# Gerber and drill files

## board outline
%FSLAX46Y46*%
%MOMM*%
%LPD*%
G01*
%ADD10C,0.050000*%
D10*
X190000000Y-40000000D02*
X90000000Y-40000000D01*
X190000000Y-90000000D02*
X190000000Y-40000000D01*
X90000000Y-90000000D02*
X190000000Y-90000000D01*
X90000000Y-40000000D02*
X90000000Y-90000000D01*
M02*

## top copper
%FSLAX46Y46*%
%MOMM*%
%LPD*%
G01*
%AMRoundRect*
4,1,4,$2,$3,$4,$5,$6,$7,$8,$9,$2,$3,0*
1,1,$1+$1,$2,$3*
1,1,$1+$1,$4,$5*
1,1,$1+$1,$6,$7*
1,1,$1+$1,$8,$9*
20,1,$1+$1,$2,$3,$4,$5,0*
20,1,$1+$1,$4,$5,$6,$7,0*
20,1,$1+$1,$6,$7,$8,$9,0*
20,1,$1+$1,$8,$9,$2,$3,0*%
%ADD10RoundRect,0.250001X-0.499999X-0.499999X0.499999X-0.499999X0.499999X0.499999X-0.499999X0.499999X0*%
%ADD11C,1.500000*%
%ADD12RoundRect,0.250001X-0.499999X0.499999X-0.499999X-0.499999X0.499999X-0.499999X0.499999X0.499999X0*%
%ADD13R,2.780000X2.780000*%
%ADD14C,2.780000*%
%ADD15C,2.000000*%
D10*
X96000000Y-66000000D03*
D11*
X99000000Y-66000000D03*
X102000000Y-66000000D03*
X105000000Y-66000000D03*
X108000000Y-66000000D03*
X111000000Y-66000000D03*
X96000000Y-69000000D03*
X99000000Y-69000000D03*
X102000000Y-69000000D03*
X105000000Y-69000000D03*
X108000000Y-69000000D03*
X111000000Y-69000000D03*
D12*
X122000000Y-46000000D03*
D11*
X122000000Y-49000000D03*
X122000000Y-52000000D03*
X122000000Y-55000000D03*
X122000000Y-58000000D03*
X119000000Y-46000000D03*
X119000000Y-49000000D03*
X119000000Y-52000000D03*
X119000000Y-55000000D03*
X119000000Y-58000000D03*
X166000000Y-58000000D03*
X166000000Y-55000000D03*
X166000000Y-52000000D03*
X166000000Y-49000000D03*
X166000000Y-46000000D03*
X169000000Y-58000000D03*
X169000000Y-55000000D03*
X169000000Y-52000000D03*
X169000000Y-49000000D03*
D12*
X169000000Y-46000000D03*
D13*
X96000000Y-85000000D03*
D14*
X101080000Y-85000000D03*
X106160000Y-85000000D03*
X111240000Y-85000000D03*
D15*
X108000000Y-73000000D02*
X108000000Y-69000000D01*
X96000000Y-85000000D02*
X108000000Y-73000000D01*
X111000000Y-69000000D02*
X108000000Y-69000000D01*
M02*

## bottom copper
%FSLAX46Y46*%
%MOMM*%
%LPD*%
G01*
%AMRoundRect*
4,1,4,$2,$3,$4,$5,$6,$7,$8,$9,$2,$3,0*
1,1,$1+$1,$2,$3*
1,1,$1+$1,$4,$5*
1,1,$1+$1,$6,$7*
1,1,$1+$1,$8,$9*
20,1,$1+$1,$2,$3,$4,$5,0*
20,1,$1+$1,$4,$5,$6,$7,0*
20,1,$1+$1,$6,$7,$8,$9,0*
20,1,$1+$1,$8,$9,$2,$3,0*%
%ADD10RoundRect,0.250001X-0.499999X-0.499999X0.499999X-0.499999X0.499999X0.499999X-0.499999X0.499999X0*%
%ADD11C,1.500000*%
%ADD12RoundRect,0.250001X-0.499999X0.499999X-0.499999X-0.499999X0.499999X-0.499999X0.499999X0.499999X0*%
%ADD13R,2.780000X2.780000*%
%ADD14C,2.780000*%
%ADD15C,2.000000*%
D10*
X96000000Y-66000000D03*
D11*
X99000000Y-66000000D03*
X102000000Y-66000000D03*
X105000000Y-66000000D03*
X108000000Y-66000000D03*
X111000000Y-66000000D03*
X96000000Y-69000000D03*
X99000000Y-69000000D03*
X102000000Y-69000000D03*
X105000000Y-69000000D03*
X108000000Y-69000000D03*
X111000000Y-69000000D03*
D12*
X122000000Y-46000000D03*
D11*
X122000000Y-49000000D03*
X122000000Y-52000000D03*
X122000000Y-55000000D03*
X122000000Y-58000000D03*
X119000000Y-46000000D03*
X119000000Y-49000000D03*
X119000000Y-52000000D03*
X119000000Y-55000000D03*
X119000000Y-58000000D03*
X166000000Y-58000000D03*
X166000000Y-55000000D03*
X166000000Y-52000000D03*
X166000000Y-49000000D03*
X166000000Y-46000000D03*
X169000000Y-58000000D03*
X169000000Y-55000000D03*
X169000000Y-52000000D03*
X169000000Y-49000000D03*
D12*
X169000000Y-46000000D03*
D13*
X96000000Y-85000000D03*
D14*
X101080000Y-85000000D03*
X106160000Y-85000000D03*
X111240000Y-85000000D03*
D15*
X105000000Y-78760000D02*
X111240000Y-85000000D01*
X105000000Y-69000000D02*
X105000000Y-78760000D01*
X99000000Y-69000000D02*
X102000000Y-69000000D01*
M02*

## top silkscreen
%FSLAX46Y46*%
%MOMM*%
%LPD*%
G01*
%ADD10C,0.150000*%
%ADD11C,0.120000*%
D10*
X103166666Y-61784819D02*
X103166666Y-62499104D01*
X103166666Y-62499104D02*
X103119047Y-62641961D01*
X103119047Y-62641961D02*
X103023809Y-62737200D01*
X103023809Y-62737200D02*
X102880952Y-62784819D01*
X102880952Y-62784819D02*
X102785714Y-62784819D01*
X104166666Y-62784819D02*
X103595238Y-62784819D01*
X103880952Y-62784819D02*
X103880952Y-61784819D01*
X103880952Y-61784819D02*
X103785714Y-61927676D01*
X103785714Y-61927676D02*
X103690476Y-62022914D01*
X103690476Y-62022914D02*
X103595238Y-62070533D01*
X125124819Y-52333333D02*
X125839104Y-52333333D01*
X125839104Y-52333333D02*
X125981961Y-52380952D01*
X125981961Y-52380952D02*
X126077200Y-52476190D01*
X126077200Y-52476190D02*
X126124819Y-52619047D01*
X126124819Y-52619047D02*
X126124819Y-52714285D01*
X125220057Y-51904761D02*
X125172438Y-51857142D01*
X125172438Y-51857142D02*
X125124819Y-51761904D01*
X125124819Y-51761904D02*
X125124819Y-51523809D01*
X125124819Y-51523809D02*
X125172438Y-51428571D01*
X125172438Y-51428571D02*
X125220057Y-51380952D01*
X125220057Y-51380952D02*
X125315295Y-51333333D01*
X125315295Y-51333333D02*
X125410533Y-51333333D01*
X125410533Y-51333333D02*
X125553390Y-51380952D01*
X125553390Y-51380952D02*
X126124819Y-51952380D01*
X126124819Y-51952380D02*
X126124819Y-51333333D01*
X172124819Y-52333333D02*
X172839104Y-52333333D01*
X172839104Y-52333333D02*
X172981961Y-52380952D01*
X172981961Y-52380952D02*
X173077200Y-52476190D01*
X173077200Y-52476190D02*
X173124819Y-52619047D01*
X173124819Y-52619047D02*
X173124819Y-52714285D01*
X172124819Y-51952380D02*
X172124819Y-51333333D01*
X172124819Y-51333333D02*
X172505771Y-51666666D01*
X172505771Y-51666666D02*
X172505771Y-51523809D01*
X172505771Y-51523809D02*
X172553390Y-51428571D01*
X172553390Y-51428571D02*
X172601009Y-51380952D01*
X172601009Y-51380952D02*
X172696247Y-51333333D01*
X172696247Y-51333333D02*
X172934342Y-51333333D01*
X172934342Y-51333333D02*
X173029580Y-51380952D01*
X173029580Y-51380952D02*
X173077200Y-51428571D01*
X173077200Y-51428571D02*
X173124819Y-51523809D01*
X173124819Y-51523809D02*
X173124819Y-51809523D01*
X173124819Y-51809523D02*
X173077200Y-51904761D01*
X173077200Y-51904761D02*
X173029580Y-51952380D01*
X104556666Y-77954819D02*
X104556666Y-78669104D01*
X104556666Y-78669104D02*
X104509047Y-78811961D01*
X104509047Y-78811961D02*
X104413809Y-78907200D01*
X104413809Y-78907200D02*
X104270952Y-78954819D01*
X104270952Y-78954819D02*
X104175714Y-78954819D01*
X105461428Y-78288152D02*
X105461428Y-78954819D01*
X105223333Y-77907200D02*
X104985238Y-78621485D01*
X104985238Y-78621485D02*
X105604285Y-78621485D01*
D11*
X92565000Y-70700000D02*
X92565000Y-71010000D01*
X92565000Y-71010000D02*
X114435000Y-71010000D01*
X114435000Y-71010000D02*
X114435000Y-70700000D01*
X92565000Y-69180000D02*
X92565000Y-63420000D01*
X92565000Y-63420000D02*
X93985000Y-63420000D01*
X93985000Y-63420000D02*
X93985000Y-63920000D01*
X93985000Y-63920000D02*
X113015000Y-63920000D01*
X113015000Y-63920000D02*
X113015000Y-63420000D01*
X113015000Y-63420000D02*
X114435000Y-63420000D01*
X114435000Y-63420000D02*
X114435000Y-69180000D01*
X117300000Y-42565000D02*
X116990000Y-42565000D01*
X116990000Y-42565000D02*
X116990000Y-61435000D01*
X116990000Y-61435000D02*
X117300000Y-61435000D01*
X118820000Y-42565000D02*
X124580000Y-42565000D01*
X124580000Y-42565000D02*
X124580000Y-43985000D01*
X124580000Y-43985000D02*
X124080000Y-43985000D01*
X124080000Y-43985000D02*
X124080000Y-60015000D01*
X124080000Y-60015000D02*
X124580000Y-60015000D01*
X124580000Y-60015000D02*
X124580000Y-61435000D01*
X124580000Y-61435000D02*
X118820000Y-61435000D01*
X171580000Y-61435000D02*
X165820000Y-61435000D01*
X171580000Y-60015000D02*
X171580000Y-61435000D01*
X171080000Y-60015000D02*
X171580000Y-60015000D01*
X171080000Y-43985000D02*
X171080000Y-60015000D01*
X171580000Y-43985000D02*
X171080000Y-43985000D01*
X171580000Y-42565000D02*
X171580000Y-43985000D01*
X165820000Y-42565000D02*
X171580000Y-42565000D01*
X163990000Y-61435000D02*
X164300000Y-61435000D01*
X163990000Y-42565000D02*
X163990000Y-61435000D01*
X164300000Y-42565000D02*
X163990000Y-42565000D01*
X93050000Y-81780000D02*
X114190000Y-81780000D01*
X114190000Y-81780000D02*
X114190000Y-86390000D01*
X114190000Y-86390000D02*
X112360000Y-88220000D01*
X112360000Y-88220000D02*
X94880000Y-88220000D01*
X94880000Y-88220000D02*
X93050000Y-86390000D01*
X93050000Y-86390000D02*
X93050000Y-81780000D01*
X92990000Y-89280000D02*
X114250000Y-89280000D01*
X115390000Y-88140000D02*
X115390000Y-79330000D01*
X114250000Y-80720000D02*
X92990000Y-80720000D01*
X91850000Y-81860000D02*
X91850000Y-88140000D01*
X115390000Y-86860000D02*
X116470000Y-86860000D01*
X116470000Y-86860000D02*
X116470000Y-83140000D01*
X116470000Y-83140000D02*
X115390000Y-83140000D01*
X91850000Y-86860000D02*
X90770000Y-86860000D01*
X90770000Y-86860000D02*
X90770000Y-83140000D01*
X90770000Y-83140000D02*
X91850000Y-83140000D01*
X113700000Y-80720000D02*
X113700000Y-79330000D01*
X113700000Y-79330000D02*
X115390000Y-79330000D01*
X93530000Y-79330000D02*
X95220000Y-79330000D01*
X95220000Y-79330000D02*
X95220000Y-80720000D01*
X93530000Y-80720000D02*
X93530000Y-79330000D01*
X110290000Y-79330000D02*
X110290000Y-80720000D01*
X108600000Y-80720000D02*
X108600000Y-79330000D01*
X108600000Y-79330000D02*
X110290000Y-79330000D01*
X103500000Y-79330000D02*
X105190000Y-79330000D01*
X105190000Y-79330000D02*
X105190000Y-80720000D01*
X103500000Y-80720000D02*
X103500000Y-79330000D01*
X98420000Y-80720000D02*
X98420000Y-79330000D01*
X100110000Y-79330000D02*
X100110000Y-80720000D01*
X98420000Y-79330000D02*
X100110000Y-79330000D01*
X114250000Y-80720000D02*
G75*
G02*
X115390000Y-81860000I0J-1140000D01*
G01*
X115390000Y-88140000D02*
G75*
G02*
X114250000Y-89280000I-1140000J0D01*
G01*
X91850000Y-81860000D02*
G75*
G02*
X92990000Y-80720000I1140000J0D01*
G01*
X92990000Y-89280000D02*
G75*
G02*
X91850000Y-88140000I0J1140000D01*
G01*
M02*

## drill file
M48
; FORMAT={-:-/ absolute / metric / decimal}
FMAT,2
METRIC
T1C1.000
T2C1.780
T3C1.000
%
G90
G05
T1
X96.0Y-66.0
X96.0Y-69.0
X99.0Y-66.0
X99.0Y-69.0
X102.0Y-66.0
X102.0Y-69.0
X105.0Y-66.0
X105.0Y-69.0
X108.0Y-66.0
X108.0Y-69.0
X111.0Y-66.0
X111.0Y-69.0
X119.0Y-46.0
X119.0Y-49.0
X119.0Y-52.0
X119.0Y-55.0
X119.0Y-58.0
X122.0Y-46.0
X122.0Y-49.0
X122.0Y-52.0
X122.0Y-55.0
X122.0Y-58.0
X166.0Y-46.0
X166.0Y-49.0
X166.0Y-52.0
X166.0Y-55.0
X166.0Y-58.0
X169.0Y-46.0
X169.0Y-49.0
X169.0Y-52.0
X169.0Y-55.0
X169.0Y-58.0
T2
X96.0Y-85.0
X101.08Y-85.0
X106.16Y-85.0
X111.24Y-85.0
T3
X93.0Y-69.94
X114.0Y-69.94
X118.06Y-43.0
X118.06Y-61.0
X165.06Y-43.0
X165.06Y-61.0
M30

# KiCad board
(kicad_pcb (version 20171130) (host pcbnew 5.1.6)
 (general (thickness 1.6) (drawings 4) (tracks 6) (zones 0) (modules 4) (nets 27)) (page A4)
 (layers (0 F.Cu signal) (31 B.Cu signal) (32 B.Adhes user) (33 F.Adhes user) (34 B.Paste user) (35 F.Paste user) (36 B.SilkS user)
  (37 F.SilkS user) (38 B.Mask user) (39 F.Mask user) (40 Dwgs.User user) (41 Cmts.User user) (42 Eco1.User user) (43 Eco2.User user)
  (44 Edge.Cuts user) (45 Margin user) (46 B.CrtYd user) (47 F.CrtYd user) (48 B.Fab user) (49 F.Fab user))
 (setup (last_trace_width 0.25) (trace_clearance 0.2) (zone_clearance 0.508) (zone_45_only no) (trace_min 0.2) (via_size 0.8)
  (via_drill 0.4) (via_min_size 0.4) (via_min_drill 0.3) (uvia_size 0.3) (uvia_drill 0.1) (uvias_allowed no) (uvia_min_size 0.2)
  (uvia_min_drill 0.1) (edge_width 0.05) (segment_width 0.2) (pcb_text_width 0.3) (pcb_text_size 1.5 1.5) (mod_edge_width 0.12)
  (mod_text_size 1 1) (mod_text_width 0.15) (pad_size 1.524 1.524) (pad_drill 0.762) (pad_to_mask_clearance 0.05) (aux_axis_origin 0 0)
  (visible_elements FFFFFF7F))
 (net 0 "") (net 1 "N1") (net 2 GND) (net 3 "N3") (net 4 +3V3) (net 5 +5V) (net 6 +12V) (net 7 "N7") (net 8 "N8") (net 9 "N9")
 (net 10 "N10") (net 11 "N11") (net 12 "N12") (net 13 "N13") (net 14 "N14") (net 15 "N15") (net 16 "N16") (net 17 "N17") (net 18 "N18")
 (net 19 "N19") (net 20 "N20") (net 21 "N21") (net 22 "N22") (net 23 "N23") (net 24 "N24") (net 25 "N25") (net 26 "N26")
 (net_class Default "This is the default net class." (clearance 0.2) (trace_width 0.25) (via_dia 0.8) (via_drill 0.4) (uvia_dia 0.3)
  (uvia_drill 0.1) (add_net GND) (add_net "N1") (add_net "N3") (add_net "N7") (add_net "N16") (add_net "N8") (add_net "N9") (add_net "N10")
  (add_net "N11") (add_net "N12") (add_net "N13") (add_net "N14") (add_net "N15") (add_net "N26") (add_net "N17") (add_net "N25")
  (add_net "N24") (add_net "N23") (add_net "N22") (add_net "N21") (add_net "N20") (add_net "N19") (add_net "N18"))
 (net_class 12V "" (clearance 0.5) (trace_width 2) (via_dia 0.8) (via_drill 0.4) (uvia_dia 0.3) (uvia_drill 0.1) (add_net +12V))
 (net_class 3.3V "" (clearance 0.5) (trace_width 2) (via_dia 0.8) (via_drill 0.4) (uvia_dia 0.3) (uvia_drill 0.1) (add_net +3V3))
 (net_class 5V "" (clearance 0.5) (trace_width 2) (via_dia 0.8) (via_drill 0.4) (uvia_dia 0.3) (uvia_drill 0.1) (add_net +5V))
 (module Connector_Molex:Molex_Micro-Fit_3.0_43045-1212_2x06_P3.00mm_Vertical (layer F.Cu) (at 96 66)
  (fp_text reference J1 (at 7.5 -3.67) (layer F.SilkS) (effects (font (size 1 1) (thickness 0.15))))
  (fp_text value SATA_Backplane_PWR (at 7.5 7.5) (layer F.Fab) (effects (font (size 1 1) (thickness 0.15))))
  (fp_line (start -3.435 4.7) (end -3.435 5.01) (layer F.SilkS) (width 0.12))
  (fp_line (start -3.435 5.01) (end 18.435 5.01) (layer F.SilkS) (width 0.12))
  (fp_line (start 18.435 5.01) (end 18.435 4.7) (layer F.SilkS) (width 0.12))
  (fp_line (start -3.435 3.18) (end -3.435 -2.58) (layer F.SilkS) (width 0.12))
  (fp_line (start -3.435 -2.58) (end -2.015 -2.58) (layer F.SilkS) (width 0.12))
  (fp_line (start -2.015 -2.58) (end -2.015 -2.08) (layer F.SilkS) (width 0.12))
  (fp_line (start -2.015 -2.08) (end 17.015 -2.08) (layer F.SilkS) (width 0.12))
  (fp_line (start 17.015 -2.08) (end 17.015 -2.58) (layer F.SilkS) (width 0.12))
  (fp_line (start 17.015 -2.58) (end 18.435 -2.58) (layer F.SilkS) (width 0.12))
  (fp_line (start 18.435 -2.58) (end 18.435 3.18) (layer F.SilkS) (width 0.12))
  (pad "" np_thru_hole circle (at -3 3.94) (size 1 1) (drill 1) (layers *.Cu *.Mask))
  (pad "" np_thru_hole circle (at 18 3.94) (size 1 1) (drill 1) (layers *.Cu *.Mask))
  (pad 1 thru_hole roundrect (at 0 0) (size 1.5 1.5) (drill 1) (layers *.Cu *.Mask) (roundrect_rratio 0.166667) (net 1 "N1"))
  (pad 2 thru_hole circle (at 3 0) (size 1.5 1.5) (drill 1) (layers *.Cu *.Mask) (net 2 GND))
  (pad 3 thru_hole circle (at 6 0) (size 1.5 1.5) (drill 1) (layers *.Cu *.Mask) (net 2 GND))
  (pad 4 thru_hole circle (at 9 0) (size 1.5 1.5) (drill 1) (layers *.Cu *.Mask) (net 2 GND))
  (pad 5 thru_hole circle (at 12 0) (size 1.5 1.5) (drill 1) (layers *.Cu *.Mask) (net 2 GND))
  (pad 6 thru_hole circle (at 15 0) (size 1.5 1.5) (drill 1) (layers *.Cu *.Mask) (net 2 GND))
  (pad 7 thru_hole circle (at 0 3) (size 1.5 1.5) (drill 1) (layers *.Cu *.Mask) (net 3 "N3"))
  (pad 8 thru_hole circle (at 3 3) (size 1.5 1.5) (drill 1) (layers *.Cu *.Mask) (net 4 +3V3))
  (pad 9 thru_hole circle (at 6 3) (size 1.5 1.5) (drill 1) (layers *.Cu *.Mask) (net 4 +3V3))
  (pad 10 thru_hole circle (at 9 3) (size 1.5 1.5) (drill 1) (layers *.Cu *.Mask) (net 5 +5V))
  (pad 11 thru_hole circle (at 12 3) (size 1.5 1.5) (drill 1) (layers *.Cu *.Mask) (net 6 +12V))
  (pad 12 thru_hole circle (at 15 3) (size 1.5 1.5) (drill 1) (layers *.Cu *.Mask) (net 6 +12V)))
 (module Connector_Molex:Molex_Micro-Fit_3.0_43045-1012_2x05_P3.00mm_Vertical (layer F.Cu) (at 122 46 270)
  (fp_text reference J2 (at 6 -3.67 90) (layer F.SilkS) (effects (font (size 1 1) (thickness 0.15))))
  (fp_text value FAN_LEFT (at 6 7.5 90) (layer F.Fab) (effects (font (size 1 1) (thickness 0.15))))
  (fp_line (start -3.435 4.7) (end -3.435 5.01) (layer F.SilkS) (width 0.12))
  (fp_line (start -3.435 5.01) (end 15.435 5.01) (layer F.SilkS) (width 0.12))
  (fp_line (start 15.435 5.01) (end 15.435 4.7) (layer F.SilkS) (width 0.12))
  (fp_line (start -3.435 3.18) (end -3.435 -2.58) (layer F.SilkS) (width 0.12))
  (fp_line (start -3.435 -2.58) (end -2.015 -2.58) (layer F.SilkS) (width 0.12))
  (fp_line (start -2.015 -2.58) (end -2.015 -2.08) (layer F.SilkS) (width 0.12))
  (fp_line (start -2.015 -2.08) (end 14.015 -2.08) (layer F.SilkS) (width 0.12))
  (fp_line (start 14.015 -2.08) (end 14.015 -2.58) (layer F.SilkS) (width 0.12))
  (fp_line (start 14.015 -2.58) (end 15.435 -2.58) (layer F.SilkS) (width 0.12))
  (fp_line (start 15.435 -2.58) (end 15.435 3.18) (layer F.SilkS) (width 0.12))
  (pad "" np_thru_hole circle (at -3 3.94 270) (size 1 1) (drill 1) (layers *.Cu *.Mask))
  (pad "" np_thru_hole circle (at 15 3.94 270) (size 1 1) (drill 1) (layers *.Cu *.Mask))
  (pad 1 thru_hole roundrect (at 0 0 270) (size 1.5 1.5) (drill 1) (layers *.Cu *.Mask) (roundrect_rratio 0.166667) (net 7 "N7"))
  (pad 2 thru_hole circle (at 3 0 270) (size 1.5 1.5) (drill 1) (layers *.Cu *.Mask) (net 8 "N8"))
  (pad 3 thru_hole circle (at 6 0 270) (size 1.5 1.5) (drill 1) (layers *.Cu *.Mask) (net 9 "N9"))
  (pad 4 thru_hole circle (at 9 0 270) (size 1.5 1.5) (drill 1) (layers *.Cu *.Mask) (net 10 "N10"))
  (pad 5 thru_hole circle (at 12 0 270) (size 1.5 1.5) (drill 1) (layers *.Cu *.Mask) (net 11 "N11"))
  (pad 6 thru_hole circle (at 0 3 270) (size 1.5 1.5) (drill 1) (layers *.Cu *.Mask) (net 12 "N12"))
  (pad 7 thru_hole circle (at 3 3 270) (size 1.5 1.5) (drill 1) (layers *.Cu *.Mask) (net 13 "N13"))
  (pad 8 thru_hole circle (at 6 3 270) (size 1.5 1.5) (drill 1) (layers *.Cu *.Mask) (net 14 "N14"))
  (pad 9 thru_hole circle (at 9 3 270) (size 1.5 1.5) (drill 1) (layers *.Cu *.Mask) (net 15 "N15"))
  (pad 10 thru_hole circle (at 12 3 270) (size 1.5 1.5) (drill 1) (layers *.Cu *.Mask) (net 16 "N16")))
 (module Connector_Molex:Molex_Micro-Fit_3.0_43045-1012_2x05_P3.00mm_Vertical (layer F.Cu) (at 169 46 270)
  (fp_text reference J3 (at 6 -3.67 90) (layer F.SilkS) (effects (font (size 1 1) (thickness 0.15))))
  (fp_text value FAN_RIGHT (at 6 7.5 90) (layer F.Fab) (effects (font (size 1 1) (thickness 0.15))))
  (fp_line (start 15.435 -2.58) (end 15.435 3.18) (layer F.SilkS) (width 0.12))
  (fp_line (start 14.015 -2.58) (end 15.435 -2.58) (layer F.SilkS) (width 0.12))
  (fp_line (start 14.015 -2.08) (end 14.015 -2.58) (layer F.SilkS) (width 0.12))
  (fp_line (start -2.015 -2.08) (end 14.015 -2.08) (layer F.SilkS) (width 0.12))
  (fp_line (start -2.015 -2.58) (end -2.015 -2.08) (layer F.SilkS) (width 0.12))
  (fp_line (start -3.435 -2.58) (end -2.015 -2.58) (layer F.SilkS) (width 0.12))
  (fp_line (start -3.435 3.18) (end -3.435 -2.58) (layer F.SilkS) (width 0.12))
  (fp_line (start 15.435 5.01) (end 15.435 4.7) (layer F.SilkS) (width 0.12))
  (fp_line (start -3.435 5.01) (end 15.435 5.01) (layer F.SilkS) (width 0.12))
  (fp_line (start -3.435 4.7) (end -3.435 5.01) (layer F.SilkS) (width 0.12))
  (pad 10 thru_hole circle (at 12 3 270) (size 1.5 1.5) (drill 1) (layers *.Cu *.Mask) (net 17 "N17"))
  (pad 9 thru_hole circle (at 9 3 270) (size 1.5 1.5) (drill 1) (layers *.Cu *.Mask) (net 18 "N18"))
  (pad 8 thru_hole circle (at 6 3 270) (size 1.5 1.5) (drill 1) (layers *.Cu *.Mask) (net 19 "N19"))
  (pad 7 thru_hole circle (at 3 3 270) (size 1.5 1.5) (drill 1) (layers *.Cu *.Mask) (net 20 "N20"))
  (pad 6 thru_hole circle (at 0 3 270) (size 1.5 1.5) (drill 1) (layers *.Cu *.Mask) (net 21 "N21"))
  (pad 5 thru_hole circle (at 12 0 270) (size 1.5 1.5) (drill 1) (layers *.Cu *.Mask) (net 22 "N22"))
  (pad 4 thru_hole circle (at 9 0 270) (size 1.5 1.5) (drill 1) (layers *.Cu *.Mask) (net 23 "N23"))
  (pad 3 thru_hole circle (at 6 0 270) (size 1.5 1.5) (drill 1) (layers *.Cu *.Mask) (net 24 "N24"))
  (pad 2 thru_hole circle (at 3 0 270) (size 1.5 1.5) (drill 1) (layers *.Cu *.Mask) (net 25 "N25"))
  (pad 1 thru_hole roundrect (at 0 0 270) (size 1.5 1.5) (drill 1) (layers *.Cu *.Mask) (roundrect_rratio 0.166667) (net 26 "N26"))
  (pad "" np_thru_hole circle (at 15 3.94 270) (size 1 1) (drill 1) (layers *.Cu *.Mask))
  (pad "" np_thru_hole circle (at -3 3.94 270) (size 1 1) (drill 1) (layers *.Cu *.Mask)))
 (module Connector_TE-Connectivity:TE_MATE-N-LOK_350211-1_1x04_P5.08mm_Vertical (layer F.Cu) (at 96 85)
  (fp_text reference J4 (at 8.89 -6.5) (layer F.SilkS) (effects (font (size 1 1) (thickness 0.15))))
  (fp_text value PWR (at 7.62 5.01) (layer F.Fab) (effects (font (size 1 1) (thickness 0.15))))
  (fp_line (start -2.95 -3.22) (end 18.19 -3.22) (layer F.SilkS) (width 0.12))
  (fp_line (start 18.19 -3.22) (end 18.19 1.39) (layer F.SilkS) (width 0.12))
  (fp_line (start 18.19 1.39) (end 16.36 3.22) (layer F.SilkS) (width 0.12))
  (fp_line (start 16.36 3.22) (end -1.12 3.22) (layer F.SilkS) (width 0.12))
  (fp_line (start -1.12 3.22) (end -2.95 1.39) (layer F.SilkS) (width 0.12))
  (fp_line (start -2.95 1.39) (end -2.95 -3.22) (layer F.SilkS) (width 0.12))
  (fp_line (start -3.01 4.28) (end 18.25 4.28) (layer F.SilkS) (width 0.12))
  (fp_line (start 19.39 3.14) (end 19.39 -5.67) (layer F.SilkS) (width 0.12))
  (fp_line (start 18.25 -4.28) (end -3.01 -4.28) (layer F.SilkS) (width 0.12))
  (fp_line (start -4.15 -3.14) (end -4.15 3.14) (layer F.SilkS) (width 0.12))
  (fp_line (start 19.39 1.86) (end 20.47 1.86) (layer F.SilkS) (width 0.12))
  (fp_line (start 20.47 1.86) (end 20.47 -1.86) (layer F.SilkS) (width 0.12))
  (fp_line (start 20.47 -1.86) (end 19.39 -1.86) (layer F.SilkS) (width 0.12))
  (fp_line (start -4.15 1.86) (end -5.23 1.86) (layer F.SilkS) (width 0.12))
  (fp_line (start -5.23 1.86) (end -5.23 -1.86) (layer F.SilkS) (width 0.12))
  (fp_line (start -5.23 -1.86) (end -4.15 -1.86) (layer F.SilkS) (width 0.12))
  (fp_line (start 17.7 -4.28) (end 17.7 -5.67) (layer F.SilkS) (width 0.12))
  (fp_line (start 17.7 -5.67) (end 19.39 -5.67) (layer F.SilkS) (width 0.12))
  (fp_line (start -2.47 -5.67) (end -0.78 -5.67) (layer F.SilkS) (width 0.12))
  (fp_line (start -0.78 -5.67) (end -0.78 -4.28) (layer F.SilkS) (width 0.12))
  (fp_line (start -2.47 -4.28) (end -2.47 -5.67) (layer F.SilkS) (width 0.12))
  (fp_line (start 14.29 -5.67) (end 14.29 -4.28) (layer F.SilkS) (width 0.12))
  (fp_line (start 12.6 -4.28) (end 12.6 -5.67) (layer F.SilkS) (width 0.12))
  (fp_line (start 12.6 -5.67) (end 14.29 -5.67) (layer F.SilkS) (width 0.12))
  (fp_line (start 7.5 -5.67) (end 9.19 -5.67) (layer F.SilkS) (width 0.12))
  (fp_line (start 9.19 -5.67) (end 9.19 -4.28) (layer F.SilkS) (width 0.12))
  (fp_line (start 7.5 -4.28) (end 7.5 -5.67) (layer F.SilkS) (width 0.12))
  (fp_line (start 2.42 -4.28) (end 2.42 -5.67) (layer F.SilkS) (width 0.12))
  (fp_line (start 4.11 -5.67) (end 4.11 -4.28) (layer F.SilkS) (width 0.12))
  (fp_line (start 2.42 -5.67) (end 4.11 -5.67) (layer F.SilkS) (width 0.12))
  (fp_arc (start 18.25 -3.14) (end 19.39 -3.14) (angle -90) (layer F.SilkS) (width 0.12))
  (fp_arc (start 18.25 3.14) (end 18.25 4.28) (angle -90) (layer F.SilkS) (width 0.12))
  (fp_arc (start -3.01 -3.14) (end -3.01 -4.28) (angle -90) (layer F.SilkS) (width 0.12))
  (fp_arc (start -3.01 3.14) (end -4.15 3.14) (angle -90) (layer F.SilkS) (width 0.12))
  (pad 1 thru_hole rect (at 0 0) (size 2.78 2.78) (drill 1.78) (layers *.Cu *.Mask) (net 6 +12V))
  (pad 2 thru_hole circle (at 5.08 0) (size 2.78 2.78) (drill 1.78) (layers *.Cu *.Mask) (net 2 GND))
  (pad 3 thru_hole circle (at 10.16 0) (size 2.78 2.78) (drill 1.78) (layers *.Cu *.Mask) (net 2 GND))
  (pad 4 thru_hole circle (at 15.24 0) (size 2.78 2.78) (drill 1.78) (layers *.Cu *.Mask) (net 5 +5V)))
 (gr_line (start 190 40) (end 90 40) (layer Edge.Cuts) (width 0.05))
 (gr_line (start 190 90) (end 190 40) (layer Edge.Cuts) (width 0.05))
 (gr_line (start 90 90) (end 190 90) (layer Edge.Cuts) (width 0.05))
 (gr_line (start 90 40) (end 90 90) (layer Edge.Cuts) (width 0.05))
 (segment (start 108 73) (end 108 69) (width 2) (layer F.Cu) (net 6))
 (segment (start 96 85) (end 108 73) (width 2) (layer F.Cu) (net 6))
 (segment (start 111 69) (end 108 69) (width 2) (layer F.Cu) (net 6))
 (segment (start 105 78.76) (end 111.24 85) (width 2) (layer B.Cu) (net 5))
 (segment (start 105 69) (end 105 78.76) (width 2) (layer B.Cu) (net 5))
 (segment (start 99 69) (end 102 69) (width 2) (layer B.Cu) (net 4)))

